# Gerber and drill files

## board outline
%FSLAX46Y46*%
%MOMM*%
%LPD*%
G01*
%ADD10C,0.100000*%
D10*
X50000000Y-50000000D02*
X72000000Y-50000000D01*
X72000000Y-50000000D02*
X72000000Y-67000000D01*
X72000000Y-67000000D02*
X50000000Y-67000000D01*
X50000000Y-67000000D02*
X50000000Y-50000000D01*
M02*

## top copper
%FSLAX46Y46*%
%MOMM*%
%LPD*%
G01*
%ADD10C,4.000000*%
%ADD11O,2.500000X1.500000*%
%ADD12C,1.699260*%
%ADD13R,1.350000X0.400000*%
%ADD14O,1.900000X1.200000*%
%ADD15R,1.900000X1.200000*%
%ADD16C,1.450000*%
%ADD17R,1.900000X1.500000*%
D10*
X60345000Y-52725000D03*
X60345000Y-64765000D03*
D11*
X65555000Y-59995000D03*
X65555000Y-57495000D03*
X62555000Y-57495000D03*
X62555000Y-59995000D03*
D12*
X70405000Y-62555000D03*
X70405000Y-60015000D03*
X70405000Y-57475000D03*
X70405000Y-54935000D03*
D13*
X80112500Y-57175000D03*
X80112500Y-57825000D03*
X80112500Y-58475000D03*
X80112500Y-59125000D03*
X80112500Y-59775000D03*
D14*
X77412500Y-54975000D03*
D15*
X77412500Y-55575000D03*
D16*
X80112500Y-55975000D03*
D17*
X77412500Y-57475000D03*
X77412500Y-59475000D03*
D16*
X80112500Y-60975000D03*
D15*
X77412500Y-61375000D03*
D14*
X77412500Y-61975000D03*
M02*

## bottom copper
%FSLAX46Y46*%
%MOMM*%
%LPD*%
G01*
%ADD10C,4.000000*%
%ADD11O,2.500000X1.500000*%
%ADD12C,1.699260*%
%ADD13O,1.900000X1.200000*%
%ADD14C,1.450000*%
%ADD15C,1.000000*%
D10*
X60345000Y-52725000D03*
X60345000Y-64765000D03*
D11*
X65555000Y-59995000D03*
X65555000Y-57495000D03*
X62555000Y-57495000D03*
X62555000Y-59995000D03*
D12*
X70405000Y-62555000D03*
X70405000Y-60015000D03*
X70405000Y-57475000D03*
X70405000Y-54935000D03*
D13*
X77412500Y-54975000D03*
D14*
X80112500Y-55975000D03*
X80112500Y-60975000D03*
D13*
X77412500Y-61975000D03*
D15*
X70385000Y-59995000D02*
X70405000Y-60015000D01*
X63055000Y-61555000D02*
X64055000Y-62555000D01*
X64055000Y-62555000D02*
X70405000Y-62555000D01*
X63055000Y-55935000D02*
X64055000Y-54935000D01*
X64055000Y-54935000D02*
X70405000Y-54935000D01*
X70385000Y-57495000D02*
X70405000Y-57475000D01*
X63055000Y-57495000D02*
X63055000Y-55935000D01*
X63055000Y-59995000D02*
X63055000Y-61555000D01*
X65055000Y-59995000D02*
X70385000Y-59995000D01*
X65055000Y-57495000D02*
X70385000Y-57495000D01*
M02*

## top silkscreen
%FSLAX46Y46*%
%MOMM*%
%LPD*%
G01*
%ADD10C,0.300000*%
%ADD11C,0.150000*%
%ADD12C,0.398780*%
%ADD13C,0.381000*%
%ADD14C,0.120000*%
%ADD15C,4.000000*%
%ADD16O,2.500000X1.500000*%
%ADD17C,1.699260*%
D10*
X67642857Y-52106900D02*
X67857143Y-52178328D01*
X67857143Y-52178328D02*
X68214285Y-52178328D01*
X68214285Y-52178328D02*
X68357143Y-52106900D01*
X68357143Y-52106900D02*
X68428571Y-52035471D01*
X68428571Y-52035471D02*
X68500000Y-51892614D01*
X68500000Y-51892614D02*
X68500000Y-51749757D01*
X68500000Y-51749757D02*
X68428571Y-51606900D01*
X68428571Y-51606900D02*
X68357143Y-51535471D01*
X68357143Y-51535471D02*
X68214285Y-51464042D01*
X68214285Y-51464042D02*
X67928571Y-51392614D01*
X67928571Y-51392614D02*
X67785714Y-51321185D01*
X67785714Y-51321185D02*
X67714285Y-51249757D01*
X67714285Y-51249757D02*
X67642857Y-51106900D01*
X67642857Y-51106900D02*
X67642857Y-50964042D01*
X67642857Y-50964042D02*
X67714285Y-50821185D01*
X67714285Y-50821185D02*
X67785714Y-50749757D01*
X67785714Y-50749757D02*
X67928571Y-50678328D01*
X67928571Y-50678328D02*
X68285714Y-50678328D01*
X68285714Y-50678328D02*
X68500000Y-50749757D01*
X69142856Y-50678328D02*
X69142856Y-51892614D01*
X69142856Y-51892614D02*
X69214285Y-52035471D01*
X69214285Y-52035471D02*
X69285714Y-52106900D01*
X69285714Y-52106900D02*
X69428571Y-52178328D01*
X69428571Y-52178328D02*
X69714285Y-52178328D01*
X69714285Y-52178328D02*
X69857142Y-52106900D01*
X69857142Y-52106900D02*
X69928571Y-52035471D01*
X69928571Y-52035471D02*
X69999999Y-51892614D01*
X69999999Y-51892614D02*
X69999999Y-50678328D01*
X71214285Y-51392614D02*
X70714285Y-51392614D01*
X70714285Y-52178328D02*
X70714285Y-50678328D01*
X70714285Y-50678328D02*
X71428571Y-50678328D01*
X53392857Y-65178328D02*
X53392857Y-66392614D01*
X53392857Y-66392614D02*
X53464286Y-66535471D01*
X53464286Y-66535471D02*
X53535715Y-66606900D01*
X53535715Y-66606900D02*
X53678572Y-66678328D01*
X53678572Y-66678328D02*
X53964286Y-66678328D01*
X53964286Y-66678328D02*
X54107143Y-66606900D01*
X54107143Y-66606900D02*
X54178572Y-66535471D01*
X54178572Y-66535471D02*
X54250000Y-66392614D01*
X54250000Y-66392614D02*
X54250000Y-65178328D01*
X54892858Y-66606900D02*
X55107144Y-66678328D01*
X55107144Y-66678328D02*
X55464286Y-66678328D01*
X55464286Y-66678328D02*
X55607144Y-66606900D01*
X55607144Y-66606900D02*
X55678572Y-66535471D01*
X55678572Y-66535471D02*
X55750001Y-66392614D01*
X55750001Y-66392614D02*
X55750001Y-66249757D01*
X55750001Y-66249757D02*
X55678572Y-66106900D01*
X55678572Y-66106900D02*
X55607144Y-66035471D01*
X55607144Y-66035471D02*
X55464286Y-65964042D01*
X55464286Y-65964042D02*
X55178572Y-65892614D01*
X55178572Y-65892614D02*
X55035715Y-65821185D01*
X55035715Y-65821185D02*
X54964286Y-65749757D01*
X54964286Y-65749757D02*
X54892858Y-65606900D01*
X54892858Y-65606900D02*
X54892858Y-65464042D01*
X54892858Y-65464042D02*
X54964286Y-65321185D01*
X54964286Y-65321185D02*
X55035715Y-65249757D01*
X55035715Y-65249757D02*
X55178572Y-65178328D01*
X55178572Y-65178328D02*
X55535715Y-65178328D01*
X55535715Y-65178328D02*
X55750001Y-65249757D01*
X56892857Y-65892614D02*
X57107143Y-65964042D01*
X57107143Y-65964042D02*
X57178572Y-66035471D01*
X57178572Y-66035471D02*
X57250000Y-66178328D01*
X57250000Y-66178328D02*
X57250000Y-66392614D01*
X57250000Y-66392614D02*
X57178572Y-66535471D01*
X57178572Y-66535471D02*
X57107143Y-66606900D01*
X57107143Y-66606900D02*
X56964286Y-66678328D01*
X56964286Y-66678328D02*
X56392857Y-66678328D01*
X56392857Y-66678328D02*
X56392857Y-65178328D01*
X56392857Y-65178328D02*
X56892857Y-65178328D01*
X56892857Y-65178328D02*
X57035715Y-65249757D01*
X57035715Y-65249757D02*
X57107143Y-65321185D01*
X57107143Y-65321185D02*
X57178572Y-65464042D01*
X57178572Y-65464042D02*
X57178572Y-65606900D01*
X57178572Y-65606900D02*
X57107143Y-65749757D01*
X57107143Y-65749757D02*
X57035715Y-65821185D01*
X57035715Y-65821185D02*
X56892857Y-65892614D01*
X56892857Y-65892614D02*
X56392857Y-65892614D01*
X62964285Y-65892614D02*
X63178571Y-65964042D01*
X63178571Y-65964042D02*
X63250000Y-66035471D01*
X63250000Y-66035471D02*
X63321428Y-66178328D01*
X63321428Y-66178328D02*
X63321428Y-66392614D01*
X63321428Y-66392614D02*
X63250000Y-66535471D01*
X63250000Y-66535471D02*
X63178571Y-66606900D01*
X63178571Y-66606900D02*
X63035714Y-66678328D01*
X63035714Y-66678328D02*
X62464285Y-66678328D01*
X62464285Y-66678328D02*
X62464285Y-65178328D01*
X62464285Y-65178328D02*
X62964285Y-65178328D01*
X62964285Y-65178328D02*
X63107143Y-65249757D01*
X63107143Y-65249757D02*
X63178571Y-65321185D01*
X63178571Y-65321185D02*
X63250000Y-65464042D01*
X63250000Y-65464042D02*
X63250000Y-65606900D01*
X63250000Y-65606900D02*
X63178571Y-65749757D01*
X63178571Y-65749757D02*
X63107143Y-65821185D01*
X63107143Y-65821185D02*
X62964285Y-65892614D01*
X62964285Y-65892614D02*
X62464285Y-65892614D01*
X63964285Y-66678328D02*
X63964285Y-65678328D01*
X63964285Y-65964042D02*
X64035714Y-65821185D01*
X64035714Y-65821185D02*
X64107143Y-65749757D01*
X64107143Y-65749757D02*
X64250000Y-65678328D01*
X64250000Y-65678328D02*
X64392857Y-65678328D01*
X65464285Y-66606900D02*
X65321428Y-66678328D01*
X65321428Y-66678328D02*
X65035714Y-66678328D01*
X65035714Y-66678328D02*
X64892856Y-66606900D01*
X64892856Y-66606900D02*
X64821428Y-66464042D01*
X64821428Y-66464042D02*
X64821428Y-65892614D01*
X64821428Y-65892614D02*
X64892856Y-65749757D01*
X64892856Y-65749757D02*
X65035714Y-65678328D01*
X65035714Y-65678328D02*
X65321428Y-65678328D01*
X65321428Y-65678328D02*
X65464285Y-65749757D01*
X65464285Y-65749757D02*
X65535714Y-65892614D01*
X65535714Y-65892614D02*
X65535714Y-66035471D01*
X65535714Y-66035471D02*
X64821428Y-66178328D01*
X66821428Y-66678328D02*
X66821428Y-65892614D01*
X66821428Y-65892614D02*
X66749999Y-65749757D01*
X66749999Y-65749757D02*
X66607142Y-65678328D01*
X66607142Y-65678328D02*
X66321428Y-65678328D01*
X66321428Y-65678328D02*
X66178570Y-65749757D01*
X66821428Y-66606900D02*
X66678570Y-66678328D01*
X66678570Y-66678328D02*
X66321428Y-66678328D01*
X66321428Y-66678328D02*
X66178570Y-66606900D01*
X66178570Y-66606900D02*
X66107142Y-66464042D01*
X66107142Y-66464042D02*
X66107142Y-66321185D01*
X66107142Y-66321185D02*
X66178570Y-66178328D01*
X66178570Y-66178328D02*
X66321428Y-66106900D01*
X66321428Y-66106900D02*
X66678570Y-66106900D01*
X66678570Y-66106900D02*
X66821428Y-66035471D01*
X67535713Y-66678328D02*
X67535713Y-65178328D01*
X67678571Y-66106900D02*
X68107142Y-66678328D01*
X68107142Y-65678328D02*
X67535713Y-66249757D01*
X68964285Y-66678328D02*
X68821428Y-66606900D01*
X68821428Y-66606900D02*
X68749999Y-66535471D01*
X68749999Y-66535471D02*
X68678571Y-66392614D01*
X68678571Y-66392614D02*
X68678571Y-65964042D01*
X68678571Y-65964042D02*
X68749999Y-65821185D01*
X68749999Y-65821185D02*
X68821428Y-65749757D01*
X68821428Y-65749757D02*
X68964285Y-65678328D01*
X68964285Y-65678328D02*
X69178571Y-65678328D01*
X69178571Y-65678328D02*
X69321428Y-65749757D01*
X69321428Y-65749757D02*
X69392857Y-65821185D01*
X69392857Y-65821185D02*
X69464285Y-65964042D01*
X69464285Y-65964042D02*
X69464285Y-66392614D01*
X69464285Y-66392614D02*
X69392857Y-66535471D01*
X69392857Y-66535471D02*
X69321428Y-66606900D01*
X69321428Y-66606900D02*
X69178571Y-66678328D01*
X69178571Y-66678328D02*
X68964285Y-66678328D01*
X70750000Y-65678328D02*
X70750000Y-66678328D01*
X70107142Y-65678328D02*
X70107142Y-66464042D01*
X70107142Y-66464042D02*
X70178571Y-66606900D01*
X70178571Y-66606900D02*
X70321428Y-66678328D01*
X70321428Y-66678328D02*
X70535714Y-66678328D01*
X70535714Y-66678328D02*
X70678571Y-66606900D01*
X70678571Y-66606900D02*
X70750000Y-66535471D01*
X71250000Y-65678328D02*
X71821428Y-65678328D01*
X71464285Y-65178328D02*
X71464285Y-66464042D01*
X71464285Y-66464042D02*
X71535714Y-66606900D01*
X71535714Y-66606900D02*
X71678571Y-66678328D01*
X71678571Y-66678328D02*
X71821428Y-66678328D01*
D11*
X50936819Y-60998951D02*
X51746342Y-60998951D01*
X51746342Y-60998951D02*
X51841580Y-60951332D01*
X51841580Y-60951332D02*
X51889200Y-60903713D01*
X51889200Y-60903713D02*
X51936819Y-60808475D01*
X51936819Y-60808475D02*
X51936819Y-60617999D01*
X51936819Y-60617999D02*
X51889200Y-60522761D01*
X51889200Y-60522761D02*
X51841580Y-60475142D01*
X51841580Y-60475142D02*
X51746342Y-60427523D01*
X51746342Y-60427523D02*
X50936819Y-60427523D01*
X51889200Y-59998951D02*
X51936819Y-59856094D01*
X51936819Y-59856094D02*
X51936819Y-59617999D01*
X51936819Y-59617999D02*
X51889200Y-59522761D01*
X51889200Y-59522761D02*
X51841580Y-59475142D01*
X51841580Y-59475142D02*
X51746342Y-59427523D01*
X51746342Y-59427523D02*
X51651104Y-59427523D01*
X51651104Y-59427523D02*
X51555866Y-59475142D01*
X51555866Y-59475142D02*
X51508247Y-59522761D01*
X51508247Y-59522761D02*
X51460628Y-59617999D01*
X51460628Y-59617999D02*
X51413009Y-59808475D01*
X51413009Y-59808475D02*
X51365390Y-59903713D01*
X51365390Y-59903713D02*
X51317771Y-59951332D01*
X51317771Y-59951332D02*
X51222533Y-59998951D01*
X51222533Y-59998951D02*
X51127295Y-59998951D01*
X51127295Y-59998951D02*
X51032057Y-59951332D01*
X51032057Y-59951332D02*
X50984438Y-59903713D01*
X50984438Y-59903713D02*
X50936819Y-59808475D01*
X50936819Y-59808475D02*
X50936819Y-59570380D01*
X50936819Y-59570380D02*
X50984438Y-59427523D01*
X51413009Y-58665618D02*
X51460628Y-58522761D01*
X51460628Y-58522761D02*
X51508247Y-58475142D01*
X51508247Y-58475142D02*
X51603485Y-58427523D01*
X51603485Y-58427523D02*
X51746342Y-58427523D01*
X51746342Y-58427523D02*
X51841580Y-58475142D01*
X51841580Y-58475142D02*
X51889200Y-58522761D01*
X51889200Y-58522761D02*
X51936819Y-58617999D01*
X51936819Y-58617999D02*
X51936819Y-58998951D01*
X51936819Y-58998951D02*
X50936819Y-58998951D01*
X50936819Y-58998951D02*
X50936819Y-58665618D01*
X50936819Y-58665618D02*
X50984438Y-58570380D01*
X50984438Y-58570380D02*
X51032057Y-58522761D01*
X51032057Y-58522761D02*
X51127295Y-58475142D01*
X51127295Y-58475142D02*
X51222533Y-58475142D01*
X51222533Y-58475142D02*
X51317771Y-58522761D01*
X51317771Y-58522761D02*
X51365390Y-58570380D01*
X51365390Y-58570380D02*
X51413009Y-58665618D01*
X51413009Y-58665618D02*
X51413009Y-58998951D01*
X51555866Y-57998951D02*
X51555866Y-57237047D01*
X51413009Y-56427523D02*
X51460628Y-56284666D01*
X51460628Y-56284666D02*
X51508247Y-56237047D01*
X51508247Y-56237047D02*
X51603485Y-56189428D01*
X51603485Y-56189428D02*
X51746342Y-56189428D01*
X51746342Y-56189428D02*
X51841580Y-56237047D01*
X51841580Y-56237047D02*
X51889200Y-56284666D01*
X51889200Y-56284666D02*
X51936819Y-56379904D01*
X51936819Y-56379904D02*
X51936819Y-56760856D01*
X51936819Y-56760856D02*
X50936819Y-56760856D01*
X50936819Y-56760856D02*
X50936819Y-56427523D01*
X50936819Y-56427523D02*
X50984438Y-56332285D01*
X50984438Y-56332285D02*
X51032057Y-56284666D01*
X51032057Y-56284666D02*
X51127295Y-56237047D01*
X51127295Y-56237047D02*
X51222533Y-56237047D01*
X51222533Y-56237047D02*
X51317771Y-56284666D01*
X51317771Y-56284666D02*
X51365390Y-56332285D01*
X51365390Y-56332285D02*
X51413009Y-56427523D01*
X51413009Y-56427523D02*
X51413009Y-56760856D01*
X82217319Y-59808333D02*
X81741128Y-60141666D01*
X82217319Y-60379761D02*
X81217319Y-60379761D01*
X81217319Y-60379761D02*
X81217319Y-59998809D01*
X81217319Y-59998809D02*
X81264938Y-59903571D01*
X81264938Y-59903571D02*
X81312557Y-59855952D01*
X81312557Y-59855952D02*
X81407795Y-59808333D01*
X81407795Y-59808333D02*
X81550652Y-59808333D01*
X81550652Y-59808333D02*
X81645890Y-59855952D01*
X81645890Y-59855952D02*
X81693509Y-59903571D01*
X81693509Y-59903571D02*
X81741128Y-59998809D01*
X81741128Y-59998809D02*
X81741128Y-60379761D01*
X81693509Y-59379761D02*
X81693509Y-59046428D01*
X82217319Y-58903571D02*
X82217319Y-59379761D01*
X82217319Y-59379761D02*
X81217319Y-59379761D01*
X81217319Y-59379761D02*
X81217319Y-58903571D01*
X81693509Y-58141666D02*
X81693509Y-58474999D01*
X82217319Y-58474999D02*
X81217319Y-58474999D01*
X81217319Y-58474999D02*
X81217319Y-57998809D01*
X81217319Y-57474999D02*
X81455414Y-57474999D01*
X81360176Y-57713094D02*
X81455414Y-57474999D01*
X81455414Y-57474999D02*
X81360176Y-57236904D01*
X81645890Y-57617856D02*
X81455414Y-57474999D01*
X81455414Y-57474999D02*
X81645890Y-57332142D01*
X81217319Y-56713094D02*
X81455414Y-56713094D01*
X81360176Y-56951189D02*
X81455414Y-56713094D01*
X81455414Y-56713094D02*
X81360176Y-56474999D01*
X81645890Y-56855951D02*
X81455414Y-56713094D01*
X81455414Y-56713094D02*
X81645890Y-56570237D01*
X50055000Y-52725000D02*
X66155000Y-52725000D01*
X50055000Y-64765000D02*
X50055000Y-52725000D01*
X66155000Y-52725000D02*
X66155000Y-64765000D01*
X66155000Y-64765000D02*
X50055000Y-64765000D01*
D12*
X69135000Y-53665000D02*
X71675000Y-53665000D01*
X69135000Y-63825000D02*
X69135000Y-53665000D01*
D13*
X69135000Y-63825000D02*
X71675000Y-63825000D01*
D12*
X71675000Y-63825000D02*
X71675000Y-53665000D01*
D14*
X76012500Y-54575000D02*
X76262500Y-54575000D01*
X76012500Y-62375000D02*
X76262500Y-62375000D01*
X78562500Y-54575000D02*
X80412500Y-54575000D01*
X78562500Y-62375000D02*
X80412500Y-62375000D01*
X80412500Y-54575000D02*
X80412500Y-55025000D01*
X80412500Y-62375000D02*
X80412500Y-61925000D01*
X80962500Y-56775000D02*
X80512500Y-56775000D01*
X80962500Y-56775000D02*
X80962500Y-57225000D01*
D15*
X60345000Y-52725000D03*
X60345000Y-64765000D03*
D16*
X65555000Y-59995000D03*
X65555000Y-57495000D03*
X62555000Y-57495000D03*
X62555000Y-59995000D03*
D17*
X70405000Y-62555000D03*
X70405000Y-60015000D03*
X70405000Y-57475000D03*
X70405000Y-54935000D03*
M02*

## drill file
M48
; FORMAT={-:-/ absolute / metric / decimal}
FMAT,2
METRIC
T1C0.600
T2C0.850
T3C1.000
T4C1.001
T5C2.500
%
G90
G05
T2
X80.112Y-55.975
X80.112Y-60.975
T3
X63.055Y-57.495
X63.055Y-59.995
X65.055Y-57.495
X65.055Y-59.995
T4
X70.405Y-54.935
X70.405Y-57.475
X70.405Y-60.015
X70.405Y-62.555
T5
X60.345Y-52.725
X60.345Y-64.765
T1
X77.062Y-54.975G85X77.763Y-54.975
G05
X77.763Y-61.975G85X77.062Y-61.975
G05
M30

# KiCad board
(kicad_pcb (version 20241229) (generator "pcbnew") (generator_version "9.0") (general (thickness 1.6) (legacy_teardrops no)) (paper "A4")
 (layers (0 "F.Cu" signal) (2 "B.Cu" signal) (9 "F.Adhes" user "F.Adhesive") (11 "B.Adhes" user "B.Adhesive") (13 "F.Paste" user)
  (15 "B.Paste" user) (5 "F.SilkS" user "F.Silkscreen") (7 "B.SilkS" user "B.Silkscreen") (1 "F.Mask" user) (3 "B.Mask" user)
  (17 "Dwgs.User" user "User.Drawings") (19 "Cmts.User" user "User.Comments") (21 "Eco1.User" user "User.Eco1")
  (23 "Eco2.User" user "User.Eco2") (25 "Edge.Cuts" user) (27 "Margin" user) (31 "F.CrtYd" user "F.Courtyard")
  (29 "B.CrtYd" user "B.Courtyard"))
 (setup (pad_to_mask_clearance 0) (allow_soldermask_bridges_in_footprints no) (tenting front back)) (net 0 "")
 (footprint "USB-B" (layer "F.Cu") (at 64.055 58.745 -90)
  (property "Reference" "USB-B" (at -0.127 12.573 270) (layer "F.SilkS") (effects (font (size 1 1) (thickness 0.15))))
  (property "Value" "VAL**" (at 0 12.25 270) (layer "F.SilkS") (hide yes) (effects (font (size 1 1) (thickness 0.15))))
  (fp_line (start -6.02 14) (end -6.02 -2.1) (stroke (width 0.15) (type solid)) (layer "F.SilkS"))
  (fp_line (start 6.02 14) (end -6.02 14) (stroke (width 0.15) (type solid)) (layer "F.SilkS"))
  (fp_line (start -6.02 -2.1) (end 6.02 -2.1) (stroke (width 0.15) (type solid)) (layer "F.SilkS"))
  (fp_line (start 6.02 -2.1) (end 6.02 14) (stroke (width 0.15) (type solid)) (layer "F.SilkS"))
  (pad "" thru_hole circle (at -6.02 3.71 270) (size 4 4) (drill 2.5) (layers "*.Cu" "*.Mask" "F.SilkS") (remove_unused_layers no))
  (pad "" thru_hole circle (at 6.02 3.71 270) (size 4 4) (drill 2.5) (layers "*.Cu" "*.Mask" "F.SilkS") (remove_unused_layers no))
  (pad "1" thru_hole oval (at 1.25 -1 270) (size 1.5 2.5) (drill 1 (offset 0 -0.5)) (layers "*.Cu" "*.Mask" "F.SilkS")
   (remove_unused_layers no))
  (pad "2" thru_hole oval (at -1.25 -1 270) (size 1.5 2.5) (drill 1 (offset 0 -0.5)) (layers "*.Cu" "*.Mask" "F.SilkS")
   (remove_unused_layers no))
  (pad "3" thru_hole oval (at -1.25 1 270) (size 1.5 2.5) (drill 1 (offset 0 0.5)) (layers "*.Cu" "*.Mask" "F.SilkS")
   (remove_unused_layers no))
  (pad "4" thru_hole oval (at 1.25 1 270) (size 1.5 2.5) (drill 1 (offset 0 0.5)) (layers "*.Cu" "*.Mask" "F.SilkS")
   (remove_unused_layers no)))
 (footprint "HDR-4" (layer "F.Cu") (at 70.405 58.745 90)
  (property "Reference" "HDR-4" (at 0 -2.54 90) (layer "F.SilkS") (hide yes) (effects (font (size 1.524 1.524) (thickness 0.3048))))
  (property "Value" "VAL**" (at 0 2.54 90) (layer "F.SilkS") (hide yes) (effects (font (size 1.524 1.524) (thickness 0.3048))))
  (fp_line (start 5.08 -1.27) (end 5.08 1.27) (stroke (width 0.39878) (type solid)) (layer "F.SilkS"))
  (fp_line (start -5.08 -1.27) (end 5.08 -1.27) (stroke (width 0.39878) (type solid)) (layer "F.SilkS"))
  (fp_line (start -5.08 -1.27) (end -5.08 1.27) (stroke (width 0.381) (type solid)) (layer "F.SilkS"))
  (fp_line (start -5.08 1.27) (end 5.08 1.27) (stroke (width 0.39878) (type solid)) (layer "F.SilkS"))
  (pad "1" thru_hole circle (at -3.81 0 90) (size 1.69926 1.69926) (drill 1.00076) (layers "*.Cu" "*.Mask" "F.SilkS")
   (remove_unused_layers no))
  (pad "2" thru_hole circle (at -1.27 0 90) (size 1.69926 1.69926) (drill 1.00076) (layers "*.Cu" "*.Mask" "F.SilkS")
   (remove_unused_layers no))
  (pad "3" thru_hole circle (at 1.27 0 90) (size 1.69926 1.69926) (drill 1.00076) (layers "*.Cu" "*.Mask" "F.SilkS")
   (remove_unused_layers no))
  (pad "4" thru_hole circle (at 3.81 0 90) (size 1.69926 1.69926) (drill 1.00076) (layers "*.Cu" "*.Mask" "F.SilkS")
   (remove_unused_layers no)))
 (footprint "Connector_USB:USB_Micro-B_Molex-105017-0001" (layer "F.Cu") (at 78.65 58.475 -90)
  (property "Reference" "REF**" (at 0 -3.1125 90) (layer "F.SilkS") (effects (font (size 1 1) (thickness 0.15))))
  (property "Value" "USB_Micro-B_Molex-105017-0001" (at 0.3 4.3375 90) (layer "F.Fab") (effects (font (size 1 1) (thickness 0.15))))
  (fp_line (start -3.9 2.6375) (end -3.9 2.3875) (stroke (width 0.12) (type solid)) (layer "F.SilkS"))
  (fp_line (start 3.9 2.6375) (end 3.9 2.3875) (stroke (width 0.12) (type solid)) (layer "F.SilkS"))
  (fp_line (start -3.9 0.0875) (end -3.9 -1.7625) (stroke (width 0.12) (type solid)) (layer "F.SilkS"))
  (fp_line (start 3.9 0.0875) (end 3.9 -1.7625) (stroke (width 0.12) (type solid)) (layer "F.SilkS"))
  (fp_line (start -3.9 -1.7625) (end -3.45 -1.7625) (stroke (width 0.12) (type solid)) (layer "F.SilkS"))
  (fp_line (start 3.9 -1.7625) (end 3.45 -1.7625) (stroke (width 0.12) (type solid)) (layer "F.SilkS"))
  (fp_line (start -1.7 -2.3125) (end -1.7 -1.8625) (stroke (width 0.12) (type solid)) (layer "F.SilkS"))
  (fp_line (start -1.7 -2.3125) (end -1.25 -2.3125) (stroke (width 0.12) (type solid)) (layer "F.SilkS"))
  (pad "1" smd rect (at -1.3 -1.4625 270) (size 0.4 1.35) (layers "F.Cu" "F.Mask" "F.Paste"))
  (pad "2" smd rect (at -0.65 -1.4625 270) (size 0.4 1.35) (layers "F.Cu" "F.Mask" "F.Paste"))
  (pad "3" smd rect (at 0 -1.4625 270) (size 0.4 1.35) (layers "F.Cu" "F.Mask" "F.Paste"))
  (pad "4" smd rect (at 0.65 -1.4625 270) (size 0.4 1.35) (layers "F.Cu" "F.Mask" "F.Paste"))
  (pad "5" smd rect (at 1.3 -1.4625 270) (size 0.4 1.35) (layers "F.Cu" "F.Mask" "F.Paste"))
  (pad "6" thru_hole oval (at -3.5 1.2375 90) (size 1.2 1.9) (drill oval 0.6 1.3) (layers "*.Cu" "*.Mask") (remove_unused_layers no))
  (pad "6" smd rect (at -2.9 1.2375 270) (size 1.2 1.9) (layers "F.Cu" "F.Mask"))
  (pad "6" thru_hole circle (at -2.5 -1.4625 270) (size 1.45 1.45) (drill 0.85) (layers "*.Cu" "*.Mask") (remove_unused_layers no))
  (pad "6" smd rect (at -1 1.2375 270) (size 1.5 1.9) (layers "F.Cu" "F.Mask" "F.Paste"))
  (pad "6" smd rect (at 1 1.2375 270) (size 1.5 1.9) (layers "F.Cu" "F.Mask" "F.Paste"))
  (pad "6" thru_hole circle (at 2.5 -1.4625 270) (size 1.45 1.45) (drill 0.85) (layers "*.Cu" "*.Mask") (remove_unused_layers no))
  (pad "6" smd rect (at 2.9 1.2375 270) (size 1.2 1.9) (layers "F.Cu" "F.Mask"))
  (pad "6" thru_hole oval (at 3.5 1.2375 270) (size 1.2 1.9) (drill oval 0.6 1.3) (layers "*.Cu" "*.Mask") (remove_unused_layers no)))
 (gr_line (start 50 50) (end 72 50) (stroke (width 0.1) (type solid)) (layer "Edge.Cuts"))
 (gr_line (start 72 50) (end 72 67) (stroke (width 0.1) (type solid)) (layer "Edge.Cuts"))
 (gr_line (start 72 67) (end 50 67) (stroke (width 0.1) (type solid)) (layer "Edge.Cuts"))
 (gr_line (start 50 67) (end 50 50) (stroke (width 0.1) (type solid)) (layer "Edge.Cuts"))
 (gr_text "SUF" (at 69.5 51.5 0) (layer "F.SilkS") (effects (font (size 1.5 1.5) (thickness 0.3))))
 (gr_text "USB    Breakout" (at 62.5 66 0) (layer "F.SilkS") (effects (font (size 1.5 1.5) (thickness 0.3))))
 (segment (start 70.385 59.995) (end 70.405 60.015) (width 1) (layer "B.Cu") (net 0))
 (segment (start 63.055 61.555) (end 64.055 62.555) (width 1) (layer "B.Cu") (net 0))
 (segment (start 64.055 62.555) (end 70.405 62.555) (width 1) (layer "B.Cu") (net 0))
 (segment (start 63.055 55.935) (end 64.055 54.935) (width 1) (layer "B.Cu") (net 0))
 (segment (start 64.055 54.935) (end 70.405 54.935) (width 1) (layer "B.Cu") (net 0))
 (segment (start 70.385 57.495) (end 70.405 57.475) (width 1) (layer "B.Cu") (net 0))
 (segment (start 63.055 57.495) (end 63.055 55.935) (width 1) (layer "B.Cu") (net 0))
 (segment (start 63.055 59.995) (end 63.055 61.555) (width 1) (layer "B.Cu") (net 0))
 (segment (start 65.055 59.995) (end 70.385 59.995) (width 1) (layer "B.Cu") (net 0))
 (segment (start 65.055 57.495) (end 70.385 57.495) (width 1) (layer "B.Cu") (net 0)))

